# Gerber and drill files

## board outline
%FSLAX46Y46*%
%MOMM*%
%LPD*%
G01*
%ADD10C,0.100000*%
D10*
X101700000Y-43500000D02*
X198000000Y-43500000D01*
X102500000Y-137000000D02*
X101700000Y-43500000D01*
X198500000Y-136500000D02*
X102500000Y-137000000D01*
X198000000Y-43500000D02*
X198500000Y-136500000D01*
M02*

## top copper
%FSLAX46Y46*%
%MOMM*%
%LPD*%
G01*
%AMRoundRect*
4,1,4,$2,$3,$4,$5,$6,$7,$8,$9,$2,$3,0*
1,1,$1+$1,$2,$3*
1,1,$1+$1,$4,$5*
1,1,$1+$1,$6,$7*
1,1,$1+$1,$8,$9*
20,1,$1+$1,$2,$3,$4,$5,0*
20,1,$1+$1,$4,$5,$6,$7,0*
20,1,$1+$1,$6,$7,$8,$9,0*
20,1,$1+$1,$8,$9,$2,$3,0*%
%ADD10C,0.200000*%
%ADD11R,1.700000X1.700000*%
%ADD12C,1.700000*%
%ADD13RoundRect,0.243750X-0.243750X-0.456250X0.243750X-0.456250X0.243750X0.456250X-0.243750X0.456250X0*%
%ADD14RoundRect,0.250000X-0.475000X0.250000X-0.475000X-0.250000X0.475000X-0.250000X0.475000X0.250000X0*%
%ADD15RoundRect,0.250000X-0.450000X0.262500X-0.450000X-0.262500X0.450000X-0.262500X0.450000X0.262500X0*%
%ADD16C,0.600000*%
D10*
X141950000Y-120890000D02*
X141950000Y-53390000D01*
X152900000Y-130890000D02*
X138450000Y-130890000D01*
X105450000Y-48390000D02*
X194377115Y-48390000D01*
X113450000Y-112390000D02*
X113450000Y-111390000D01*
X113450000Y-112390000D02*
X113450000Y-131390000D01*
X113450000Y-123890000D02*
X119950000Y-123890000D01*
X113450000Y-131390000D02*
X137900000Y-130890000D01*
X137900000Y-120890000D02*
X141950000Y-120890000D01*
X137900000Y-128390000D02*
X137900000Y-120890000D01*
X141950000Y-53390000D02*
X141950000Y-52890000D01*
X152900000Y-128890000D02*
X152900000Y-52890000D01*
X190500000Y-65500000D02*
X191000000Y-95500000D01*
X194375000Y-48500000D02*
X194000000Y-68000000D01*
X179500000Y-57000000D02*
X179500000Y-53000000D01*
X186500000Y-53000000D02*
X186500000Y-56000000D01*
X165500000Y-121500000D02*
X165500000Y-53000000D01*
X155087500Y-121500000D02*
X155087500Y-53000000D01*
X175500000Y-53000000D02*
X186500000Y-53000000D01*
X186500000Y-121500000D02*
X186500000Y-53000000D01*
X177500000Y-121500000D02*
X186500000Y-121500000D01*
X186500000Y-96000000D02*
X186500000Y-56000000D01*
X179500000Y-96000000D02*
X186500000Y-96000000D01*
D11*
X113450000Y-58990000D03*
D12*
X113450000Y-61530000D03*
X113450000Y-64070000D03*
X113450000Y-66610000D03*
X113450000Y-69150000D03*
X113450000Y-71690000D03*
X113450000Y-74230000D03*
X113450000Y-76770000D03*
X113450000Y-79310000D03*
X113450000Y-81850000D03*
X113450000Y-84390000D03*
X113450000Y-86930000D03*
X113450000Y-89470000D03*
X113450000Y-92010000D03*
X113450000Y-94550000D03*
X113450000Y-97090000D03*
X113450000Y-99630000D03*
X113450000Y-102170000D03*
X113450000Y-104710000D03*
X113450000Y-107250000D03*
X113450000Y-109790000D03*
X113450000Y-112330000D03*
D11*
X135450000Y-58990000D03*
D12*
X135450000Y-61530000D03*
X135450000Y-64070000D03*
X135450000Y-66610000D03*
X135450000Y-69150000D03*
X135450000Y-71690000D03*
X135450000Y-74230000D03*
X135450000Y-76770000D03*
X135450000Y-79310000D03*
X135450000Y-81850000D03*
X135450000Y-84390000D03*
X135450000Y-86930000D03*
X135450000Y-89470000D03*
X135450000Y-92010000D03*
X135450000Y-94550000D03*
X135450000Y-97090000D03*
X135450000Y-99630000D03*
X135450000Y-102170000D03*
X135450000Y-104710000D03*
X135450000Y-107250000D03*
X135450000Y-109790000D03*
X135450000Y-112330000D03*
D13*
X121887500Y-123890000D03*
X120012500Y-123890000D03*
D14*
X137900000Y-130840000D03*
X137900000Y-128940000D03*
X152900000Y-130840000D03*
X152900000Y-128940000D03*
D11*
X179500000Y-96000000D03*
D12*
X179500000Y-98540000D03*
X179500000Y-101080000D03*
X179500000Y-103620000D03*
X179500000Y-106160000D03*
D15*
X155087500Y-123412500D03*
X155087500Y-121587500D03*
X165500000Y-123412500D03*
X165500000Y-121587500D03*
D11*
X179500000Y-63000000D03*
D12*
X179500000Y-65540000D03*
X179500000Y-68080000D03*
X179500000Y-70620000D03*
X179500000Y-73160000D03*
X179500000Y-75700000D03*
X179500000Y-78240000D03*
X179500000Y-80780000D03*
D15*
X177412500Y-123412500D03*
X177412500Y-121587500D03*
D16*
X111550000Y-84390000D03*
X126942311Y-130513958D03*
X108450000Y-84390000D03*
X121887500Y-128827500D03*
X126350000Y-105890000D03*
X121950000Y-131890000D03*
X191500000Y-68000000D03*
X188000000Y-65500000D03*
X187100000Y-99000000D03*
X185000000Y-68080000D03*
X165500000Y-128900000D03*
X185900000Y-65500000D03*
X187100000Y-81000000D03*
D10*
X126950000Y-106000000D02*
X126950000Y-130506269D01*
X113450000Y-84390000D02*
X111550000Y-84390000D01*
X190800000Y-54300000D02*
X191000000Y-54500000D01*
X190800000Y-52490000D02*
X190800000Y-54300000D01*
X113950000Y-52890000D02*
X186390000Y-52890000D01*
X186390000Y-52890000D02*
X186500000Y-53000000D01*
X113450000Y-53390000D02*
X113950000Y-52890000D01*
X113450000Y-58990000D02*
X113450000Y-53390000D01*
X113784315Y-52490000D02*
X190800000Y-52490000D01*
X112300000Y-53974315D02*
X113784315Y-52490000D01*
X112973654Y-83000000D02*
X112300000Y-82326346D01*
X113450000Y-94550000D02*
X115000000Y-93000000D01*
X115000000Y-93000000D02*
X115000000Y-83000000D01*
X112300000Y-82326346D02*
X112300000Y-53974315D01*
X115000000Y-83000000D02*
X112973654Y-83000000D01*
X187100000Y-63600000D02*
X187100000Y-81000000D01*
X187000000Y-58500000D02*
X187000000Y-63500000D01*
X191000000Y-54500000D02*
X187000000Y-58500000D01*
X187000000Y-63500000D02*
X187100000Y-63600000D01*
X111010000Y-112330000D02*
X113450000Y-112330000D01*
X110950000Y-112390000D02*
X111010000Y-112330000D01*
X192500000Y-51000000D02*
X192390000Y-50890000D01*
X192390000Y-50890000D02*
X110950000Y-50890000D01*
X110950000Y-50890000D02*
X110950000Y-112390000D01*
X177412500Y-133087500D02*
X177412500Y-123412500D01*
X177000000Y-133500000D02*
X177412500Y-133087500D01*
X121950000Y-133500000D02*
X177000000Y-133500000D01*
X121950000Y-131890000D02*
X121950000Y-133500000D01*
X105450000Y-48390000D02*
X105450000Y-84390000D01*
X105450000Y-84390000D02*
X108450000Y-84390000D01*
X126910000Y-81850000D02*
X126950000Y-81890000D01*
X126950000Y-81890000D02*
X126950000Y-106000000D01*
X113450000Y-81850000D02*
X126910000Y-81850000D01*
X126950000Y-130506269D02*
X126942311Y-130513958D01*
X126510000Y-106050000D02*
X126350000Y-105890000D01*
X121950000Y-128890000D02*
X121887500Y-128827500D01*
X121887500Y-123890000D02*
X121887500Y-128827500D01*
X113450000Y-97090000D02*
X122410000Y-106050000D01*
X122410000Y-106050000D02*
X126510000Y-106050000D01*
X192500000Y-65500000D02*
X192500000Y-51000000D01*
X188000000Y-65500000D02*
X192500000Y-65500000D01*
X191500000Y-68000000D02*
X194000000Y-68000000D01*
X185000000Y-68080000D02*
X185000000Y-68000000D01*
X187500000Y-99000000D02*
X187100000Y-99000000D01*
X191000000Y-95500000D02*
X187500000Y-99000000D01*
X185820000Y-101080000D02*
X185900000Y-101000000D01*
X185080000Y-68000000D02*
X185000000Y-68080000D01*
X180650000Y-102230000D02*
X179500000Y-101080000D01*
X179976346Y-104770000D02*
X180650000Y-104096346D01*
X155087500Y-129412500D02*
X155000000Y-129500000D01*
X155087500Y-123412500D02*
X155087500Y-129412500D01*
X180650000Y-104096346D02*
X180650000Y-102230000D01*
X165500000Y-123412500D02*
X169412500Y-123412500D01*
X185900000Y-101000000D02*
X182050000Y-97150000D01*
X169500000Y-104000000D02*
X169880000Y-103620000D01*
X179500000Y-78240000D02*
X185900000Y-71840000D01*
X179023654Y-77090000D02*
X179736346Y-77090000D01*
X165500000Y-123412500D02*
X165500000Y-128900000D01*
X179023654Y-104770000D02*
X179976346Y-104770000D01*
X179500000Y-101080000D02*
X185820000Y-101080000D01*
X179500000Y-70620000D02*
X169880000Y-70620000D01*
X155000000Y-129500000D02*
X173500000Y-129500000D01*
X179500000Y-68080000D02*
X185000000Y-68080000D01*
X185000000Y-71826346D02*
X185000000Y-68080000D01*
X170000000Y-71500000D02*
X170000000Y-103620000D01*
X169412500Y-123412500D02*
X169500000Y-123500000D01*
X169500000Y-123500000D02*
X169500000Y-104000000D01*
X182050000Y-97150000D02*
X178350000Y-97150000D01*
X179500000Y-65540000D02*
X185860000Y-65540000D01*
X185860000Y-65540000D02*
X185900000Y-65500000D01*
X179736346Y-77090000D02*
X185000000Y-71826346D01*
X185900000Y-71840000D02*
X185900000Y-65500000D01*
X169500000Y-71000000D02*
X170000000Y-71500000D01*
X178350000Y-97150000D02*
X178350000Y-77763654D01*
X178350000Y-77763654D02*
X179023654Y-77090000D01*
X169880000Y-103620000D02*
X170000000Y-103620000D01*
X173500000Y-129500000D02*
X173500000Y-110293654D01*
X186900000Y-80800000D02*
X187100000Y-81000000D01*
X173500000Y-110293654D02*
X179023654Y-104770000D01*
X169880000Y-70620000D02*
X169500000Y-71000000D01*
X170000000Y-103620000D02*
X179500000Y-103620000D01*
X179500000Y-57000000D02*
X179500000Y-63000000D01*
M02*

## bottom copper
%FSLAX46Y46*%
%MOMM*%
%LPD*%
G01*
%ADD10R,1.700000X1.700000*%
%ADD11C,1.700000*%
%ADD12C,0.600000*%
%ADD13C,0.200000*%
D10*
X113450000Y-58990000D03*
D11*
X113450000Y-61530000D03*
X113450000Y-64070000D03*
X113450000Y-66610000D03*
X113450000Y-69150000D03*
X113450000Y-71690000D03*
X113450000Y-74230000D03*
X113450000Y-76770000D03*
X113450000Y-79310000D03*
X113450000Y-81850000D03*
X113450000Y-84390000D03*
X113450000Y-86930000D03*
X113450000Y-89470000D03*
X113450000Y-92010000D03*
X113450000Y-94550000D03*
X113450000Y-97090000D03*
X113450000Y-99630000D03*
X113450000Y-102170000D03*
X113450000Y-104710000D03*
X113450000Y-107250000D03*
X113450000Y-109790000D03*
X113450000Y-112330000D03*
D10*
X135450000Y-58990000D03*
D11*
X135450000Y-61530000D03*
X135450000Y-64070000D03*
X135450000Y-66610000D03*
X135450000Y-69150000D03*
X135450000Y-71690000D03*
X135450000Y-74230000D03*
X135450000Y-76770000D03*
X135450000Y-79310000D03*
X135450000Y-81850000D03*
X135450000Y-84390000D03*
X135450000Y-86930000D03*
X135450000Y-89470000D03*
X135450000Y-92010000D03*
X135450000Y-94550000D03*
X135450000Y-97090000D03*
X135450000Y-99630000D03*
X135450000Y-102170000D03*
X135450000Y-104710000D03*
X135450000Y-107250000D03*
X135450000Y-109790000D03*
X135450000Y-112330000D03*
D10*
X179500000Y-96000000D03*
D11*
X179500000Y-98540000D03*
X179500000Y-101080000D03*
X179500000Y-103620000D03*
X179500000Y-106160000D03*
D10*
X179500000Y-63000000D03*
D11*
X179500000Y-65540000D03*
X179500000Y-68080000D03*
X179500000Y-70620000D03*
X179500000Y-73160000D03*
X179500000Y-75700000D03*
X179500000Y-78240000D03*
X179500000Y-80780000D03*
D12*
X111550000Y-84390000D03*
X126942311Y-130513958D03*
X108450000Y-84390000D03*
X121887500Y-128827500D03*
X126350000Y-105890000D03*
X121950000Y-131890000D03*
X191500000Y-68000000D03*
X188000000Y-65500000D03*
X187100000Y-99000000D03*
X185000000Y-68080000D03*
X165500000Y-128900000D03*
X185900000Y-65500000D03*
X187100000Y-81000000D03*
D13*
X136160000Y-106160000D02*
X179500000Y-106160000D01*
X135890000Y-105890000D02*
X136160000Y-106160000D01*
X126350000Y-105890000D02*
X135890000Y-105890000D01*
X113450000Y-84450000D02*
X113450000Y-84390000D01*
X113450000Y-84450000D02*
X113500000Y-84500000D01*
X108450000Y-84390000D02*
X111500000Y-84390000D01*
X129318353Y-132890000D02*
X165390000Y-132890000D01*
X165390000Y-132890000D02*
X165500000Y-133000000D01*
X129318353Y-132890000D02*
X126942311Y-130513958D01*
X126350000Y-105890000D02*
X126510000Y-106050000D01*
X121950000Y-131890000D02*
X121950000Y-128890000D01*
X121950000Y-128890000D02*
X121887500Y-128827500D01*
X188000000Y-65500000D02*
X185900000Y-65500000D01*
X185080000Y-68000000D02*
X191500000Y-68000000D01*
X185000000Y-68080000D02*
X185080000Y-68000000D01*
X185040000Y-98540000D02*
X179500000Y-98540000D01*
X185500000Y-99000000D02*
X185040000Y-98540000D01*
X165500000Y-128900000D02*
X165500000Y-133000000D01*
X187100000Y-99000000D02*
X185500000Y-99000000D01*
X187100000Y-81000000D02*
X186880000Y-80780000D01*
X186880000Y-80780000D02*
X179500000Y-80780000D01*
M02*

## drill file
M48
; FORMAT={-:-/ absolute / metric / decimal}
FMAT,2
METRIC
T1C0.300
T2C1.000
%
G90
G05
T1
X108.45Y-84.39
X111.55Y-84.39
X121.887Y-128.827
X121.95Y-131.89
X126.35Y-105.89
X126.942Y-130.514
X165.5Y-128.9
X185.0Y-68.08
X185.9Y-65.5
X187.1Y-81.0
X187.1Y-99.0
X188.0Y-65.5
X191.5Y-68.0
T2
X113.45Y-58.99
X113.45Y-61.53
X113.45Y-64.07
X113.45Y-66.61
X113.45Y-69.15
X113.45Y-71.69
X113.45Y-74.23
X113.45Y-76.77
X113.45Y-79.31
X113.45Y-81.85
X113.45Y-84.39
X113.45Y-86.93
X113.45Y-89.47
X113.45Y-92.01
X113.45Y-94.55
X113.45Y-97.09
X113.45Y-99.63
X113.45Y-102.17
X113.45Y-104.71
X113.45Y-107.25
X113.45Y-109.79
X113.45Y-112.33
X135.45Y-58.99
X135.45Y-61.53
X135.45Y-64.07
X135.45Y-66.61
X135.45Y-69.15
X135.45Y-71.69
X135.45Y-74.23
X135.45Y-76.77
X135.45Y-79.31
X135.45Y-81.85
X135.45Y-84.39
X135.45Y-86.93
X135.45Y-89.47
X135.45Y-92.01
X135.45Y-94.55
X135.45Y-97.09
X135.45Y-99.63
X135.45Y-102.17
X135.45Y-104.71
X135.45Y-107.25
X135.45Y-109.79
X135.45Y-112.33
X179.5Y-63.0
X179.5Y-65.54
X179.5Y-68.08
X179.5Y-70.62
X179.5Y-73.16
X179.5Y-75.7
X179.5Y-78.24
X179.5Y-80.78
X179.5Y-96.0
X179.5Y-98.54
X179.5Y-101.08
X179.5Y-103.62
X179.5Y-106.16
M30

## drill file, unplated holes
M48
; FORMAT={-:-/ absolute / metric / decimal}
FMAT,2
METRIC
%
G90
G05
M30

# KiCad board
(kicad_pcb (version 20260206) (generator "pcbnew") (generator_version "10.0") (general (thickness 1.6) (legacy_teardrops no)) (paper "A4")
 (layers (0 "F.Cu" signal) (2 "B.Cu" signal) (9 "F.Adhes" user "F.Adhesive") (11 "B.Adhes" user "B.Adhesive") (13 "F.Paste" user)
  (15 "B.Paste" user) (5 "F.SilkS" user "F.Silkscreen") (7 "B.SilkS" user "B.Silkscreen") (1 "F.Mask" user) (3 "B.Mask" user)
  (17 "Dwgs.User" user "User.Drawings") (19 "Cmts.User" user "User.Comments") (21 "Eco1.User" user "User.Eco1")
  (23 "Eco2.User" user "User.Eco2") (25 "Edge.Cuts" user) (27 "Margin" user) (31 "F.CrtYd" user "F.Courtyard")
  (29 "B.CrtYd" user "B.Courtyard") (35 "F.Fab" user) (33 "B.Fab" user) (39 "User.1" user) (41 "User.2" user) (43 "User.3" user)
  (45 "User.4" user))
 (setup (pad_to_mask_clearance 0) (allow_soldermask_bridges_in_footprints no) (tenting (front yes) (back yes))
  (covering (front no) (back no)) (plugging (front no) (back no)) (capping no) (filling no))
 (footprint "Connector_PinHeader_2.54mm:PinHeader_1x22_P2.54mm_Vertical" (layer "F.Cu") (at 135.45 58.99)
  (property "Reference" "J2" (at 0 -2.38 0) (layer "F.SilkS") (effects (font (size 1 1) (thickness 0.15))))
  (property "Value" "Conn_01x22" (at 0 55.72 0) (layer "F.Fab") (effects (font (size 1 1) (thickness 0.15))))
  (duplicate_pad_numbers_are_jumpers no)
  (pad "1" thru_hole rect (at 0 0) (size 1.7 1.7) (drill 1) (layers "*.Cu" "*.Mask") (remove_unused_layers no)
   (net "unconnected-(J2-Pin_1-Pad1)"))
  (pad "2" thru_hole circle (at 0 2.54) (size 1.7 1.7) (drill 1) (layers "*.Cu" "*.Mask") (remove_unused_layers no)
   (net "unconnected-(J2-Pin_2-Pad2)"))
  (pad "3" thru_hole circle (at 0 5.08) (size 1.7 1.7) (drill 1) (layers "*.Cu" "*.Mask") (remove_unused_layers no)
   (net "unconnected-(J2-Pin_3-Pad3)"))
  (pad "4" thru_hole circle (at 0 7.62) (size 1.7 1.7) (drill 1) (layers "*.Cu" "*.Mask") (remove_unused_layers no)
   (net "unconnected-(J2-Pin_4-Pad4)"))
  (pad "5" thru_hole circle (at 0 10.16) (size 1.7 1.7) (drill 1) (layers "*.Cu" "*.Mask") (remove_unused_layers no)
   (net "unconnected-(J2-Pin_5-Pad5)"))
  (pad "6" thru_hole circle (at 0 12.7) (size 1.7 1.7) (drill 1) (layers "*.Cu" "*.Mask") (remove_unused_layers no)
   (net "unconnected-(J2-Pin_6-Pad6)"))
  (pad "7" thru_hole circle (at 0 15.24) (size 1.7 1.7) (drill 1) (layers "*.Cu" "*.Mask") (remove_unused_layers no)
   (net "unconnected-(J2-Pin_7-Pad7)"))
  (pad "8" thru_hole circle (at 0 17.78) (size 1.7 1.7) (drill 1) (layers "*.Cu" "*.Mask") (remove_unused_layers no)
   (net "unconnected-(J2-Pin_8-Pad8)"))
  (pad "9" thru_hole circle (at 0 20.32) (size 1.7 1.7) (drill 1) (layers "*.Cu" "*.Mask") (remove_unused_layers no)
   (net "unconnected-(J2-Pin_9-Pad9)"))
  (pad "10" thru_hole circle (at 0 22.86) (size 1.7 1.7) (drill 1) (layers "*.Cu" "*.Mask") (remove_unused_layers no)
   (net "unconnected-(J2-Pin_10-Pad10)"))
  (pad "11" thru_hole circle (at 0 25.4) (size 1.7 1.7) (drill 1) (layers "*.Cu" "*.Mask") (remove_unused_layers no)
   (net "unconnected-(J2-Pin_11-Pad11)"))
  (pad "12" thru_hole circle (at 0 27.94) (size 1.7 1.7) (drill 1) (layers "*.Cu" "*.Mask") (remove_unused_layers no)
   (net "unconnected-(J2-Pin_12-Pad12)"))
  (pad "13" thru_hole circle (at 0 30.48) (size 1.7 1.7) (drill 1) (layers "*.Cu" "*.Mask") (remove_unused_layers no)
   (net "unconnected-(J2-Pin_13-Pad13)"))
  (pad "14" thru_hole circle (at 0 33.02) (size 1.7 1.7) (drill 1) (layers "*.Cu" "*.Mask") (remove_unused_layers no)
   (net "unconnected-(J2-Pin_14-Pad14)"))
  (pad "15" thru_hole circle (at 0 35.56) (size 1.7 1.7) (drill 1) (layers "*.Cu" "*.Mask") (remove_unused_layers no)
   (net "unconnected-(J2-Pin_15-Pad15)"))
  (pad "16" thru_hole circle (at 0 38.1) (size 1.7 1.7) (drill 1) (layers "*.Cu" "*.Mask") (remove_unused_layers no)
   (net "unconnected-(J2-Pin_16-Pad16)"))
  (pad "17" thru_hole circle (at 0 40.64) (size 1.7 1.7) (drill 1) (layers "*.Cu" "*.Mask") (remove_unused_layers no)
   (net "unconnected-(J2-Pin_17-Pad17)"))
  (pad "18" thru_hole circle (at 0 43.18) (size 1.7 1.7) (drill 1) (layers "*.Cu" "*.Mask") (remove_unused_layers no)
   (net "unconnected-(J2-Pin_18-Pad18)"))
  (pad "19" thru_hole circle (at 0 45.72) (size 1.7 1.7) (drill 1) (layers "*.Cu" "*.Mask") (remove_unused_layers no)
   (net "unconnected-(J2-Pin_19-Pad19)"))
  (pad "20" thru_hole circle (at 0 48.26) (size 1.7 1.7) (drill 1) (layers "*.Cu" "*.Mask") (remove_unused_layers no)
   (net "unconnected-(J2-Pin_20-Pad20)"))
  (pad "21" thru_hole circle (at 0 50.8) (size 1.7 1.7) (drill 1) (layers "*.Cu" "*.Mask") (remove_unused_layers no)
   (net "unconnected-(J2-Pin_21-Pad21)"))
  (pad "22" thru_hole circle (at 0 53.34) (size 1.7 1.7) (drill 1) (layers "*.Cu" "*.Mask") (remove_unused_layers no)
   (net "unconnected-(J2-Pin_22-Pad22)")))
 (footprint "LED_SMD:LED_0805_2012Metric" (layer "F.Cu") (at 120.95 123.89)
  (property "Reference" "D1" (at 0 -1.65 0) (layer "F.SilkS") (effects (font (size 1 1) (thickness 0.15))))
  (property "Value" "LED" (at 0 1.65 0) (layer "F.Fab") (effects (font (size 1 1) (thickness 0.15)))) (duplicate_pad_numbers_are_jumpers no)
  (pad "1" smd roundrect (at -0.9375 0) (size 0.975 1.4) (layers "F.Cu" "F.Mask" "F.Paste") (roundrect_rratio 0.25) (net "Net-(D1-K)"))
  (pad "2" smd roundrect (at 0.9375 0) (size 0.975 1.4) (layers "F.Cu" "F.Mask" "F.Paste") (roundrect_rratio 0.25) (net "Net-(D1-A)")))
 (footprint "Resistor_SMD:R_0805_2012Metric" (layer "F.Cu") (at 165.5 122.5 -90)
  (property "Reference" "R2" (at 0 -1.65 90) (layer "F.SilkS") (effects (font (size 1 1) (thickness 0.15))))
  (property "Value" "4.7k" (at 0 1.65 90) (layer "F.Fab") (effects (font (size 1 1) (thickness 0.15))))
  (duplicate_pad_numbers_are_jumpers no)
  (pad "1" smd roundrect (at -0.9125 0 270) (size 1.025 1.4) (layers "F.Cu" "F.Mask" "F.Paste") (roundrect_rratio 0.243902) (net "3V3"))
  (pad "2" smd roundrect (at 0.9125 0 270) (size 1.025 1.4) (layers "F.Cu" "F.Mask" "F.Paste") (roundrect_rratio 0.243902)
   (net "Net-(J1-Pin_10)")))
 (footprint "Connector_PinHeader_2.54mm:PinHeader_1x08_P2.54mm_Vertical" (layer "F.Cu") (at 179.5 63)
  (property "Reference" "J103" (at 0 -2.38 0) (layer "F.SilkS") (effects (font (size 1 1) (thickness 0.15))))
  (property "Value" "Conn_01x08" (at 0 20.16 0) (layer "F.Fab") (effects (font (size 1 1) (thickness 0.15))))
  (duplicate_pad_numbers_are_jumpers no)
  (pad "1" thru_hole rect (at 0 0) (size 1.7 1.7) (drill 1) (layers "*.Cu" "*.Mask") (remove_unused_layers no) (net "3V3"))
  (pad "2" thru_hole circle (at 0 2.54) (size 1.7 1.7) (drill 1) (layers "*.Cu" "*.Mask") (remove_unused_layers no) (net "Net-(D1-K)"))
  (pad "3" thru_hole circle (at 0 5.08) (size 1.7 1.7) (drill 1) (layers "*.Cu" "*.Mask") (remove_unused_layers no) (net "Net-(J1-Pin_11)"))
  (pad "4" thru_hole circle (at 0 7.62) (size 1.7 1.7) (drill 1) (layers "*.Cu" "*.Mask") (remove_unused_layers no) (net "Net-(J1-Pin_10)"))
  (pad "5" thru_hole circle (at 0 10.16) (size 1.7 1.7) (drill 1) (layers "*.Cu" "*.Mask") (remove_unused_layers no)
   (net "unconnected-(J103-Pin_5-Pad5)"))
  (pad "6" thru_hole circle (at 0 12.7) (size 1.7 1.7) (drill 1) (layers "*.Cu" "*.Mask") (remove_unused_layers no)
   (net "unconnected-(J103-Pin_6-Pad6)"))
  (pad "7" thru_hole circle (at 0 15.24) (size 1.7 1.7) (drill 1) (layers "*.Cu" "*.Mask") (remove_unused_layers no) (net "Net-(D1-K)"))
  (pad "8" thru_hole circle (at 0 17.78) (size 1.7 1.7) (drill 1) (layers "*.Cu" "*.Mask") (remove_unused_layers no) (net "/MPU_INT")))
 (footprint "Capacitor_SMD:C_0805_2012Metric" (layer "F.Cu") (at 137.9 129.89 -90)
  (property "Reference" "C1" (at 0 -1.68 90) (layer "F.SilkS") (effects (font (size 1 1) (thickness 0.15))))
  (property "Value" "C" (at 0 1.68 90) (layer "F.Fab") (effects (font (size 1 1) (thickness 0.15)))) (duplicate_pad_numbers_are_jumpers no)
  (pad "1" smd roundrect (at -0.95 0 270) (size 1 1.45) (layers "F.Cu" "F.Mask" "F.Paste") (roundrect_rratio 0.25) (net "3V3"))
  (pad "2" smd roundrect (at 0.95 0 270) (size 1 1.45) (layers "F.Cu" "F.Mask" "F.Paste") (roundrect_rratio 0.25) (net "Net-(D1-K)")))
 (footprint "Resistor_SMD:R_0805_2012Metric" (layer "F.Cu") (at 177.4125 122.5 -90)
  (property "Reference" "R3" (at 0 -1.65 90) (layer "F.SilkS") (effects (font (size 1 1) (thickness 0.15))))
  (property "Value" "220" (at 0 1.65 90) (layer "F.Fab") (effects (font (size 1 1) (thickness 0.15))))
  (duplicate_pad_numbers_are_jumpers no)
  (pad "1" smd roundrect (at -0.9125 0 270) (size 1.025 1.4) (layers "F.Cu" "F.Mask" "F.Paste") (roundrect_rratio 0.243902) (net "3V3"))
  (pad "2" smd roundrect (at 0.9125 0 270) (size 1.025 1.4) (layers "F.Cu" "F.Mask" "F.Paste") (roundrect_rratio 0.243902)
   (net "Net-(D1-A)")))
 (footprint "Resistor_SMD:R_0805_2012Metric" (layer "F.Cu") (at 155.0875 122.5 -90)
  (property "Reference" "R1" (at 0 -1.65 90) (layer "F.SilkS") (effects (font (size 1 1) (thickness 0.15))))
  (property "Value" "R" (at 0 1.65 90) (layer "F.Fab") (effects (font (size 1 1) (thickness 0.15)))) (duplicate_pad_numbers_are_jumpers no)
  (pad "1" smd roundrect (at -0.9125 0 270) (size 1.025 1.4) (layers "F.Cu" "F.Mask" "F.Paste") (roundrect_rratio 0.243902) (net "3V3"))
  (pad "2" smd roundrect (at 0.9125 0 270) (size 1.025 1.4) (layers "F.Cu" "F.Mask" "F.Paste") (roundrect_rratio 0.243902)
   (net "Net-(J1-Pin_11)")))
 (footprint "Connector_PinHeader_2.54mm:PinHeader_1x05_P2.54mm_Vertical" (layer "F.Cu") (at 179.5 96)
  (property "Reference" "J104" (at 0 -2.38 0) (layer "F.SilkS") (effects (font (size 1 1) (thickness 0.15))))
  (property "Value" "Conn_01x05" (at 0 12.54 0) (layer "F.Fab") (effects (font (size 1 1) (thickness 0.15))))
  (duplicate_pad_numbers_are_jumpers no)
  (pad "1" thru_hole rect (at 0 0) (size 1.7 1.7) (drill 1) (layers "*.Cu" "*.Mask") (remove_unused_layers no) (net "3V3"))
  (pad "2" thru_hole circle (at 0 2.54) (size 1.7 1.7) (drill 1) (layers "*.Cu" "*.Mask") (remove_unused_layers no) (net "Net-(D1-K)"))
  (pad "3" thru_hole circle (at 0 5.08) (size 1.7 1.7) (drill 1) (layers "*.Cu" "*.Mask") (remove_unused_layers no) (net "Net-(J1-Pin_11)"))
  (pad "4" thru_hole circle (at 0 7.62) (size 1.7 1.7) (drill 1) (layers "*.Cu" "*.Mask") (remove_unused_layers no) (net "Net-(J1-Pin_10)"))
  (pad "5" thru_hole circle (at 0 10.16) (size 1.7 1.7) (drill 1) (layers "*.Cu" "*.Mask") (remove_unused_layers no) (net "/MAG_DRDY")))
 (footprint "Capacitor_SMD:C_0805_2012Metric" (layer "F.Cu") (at 152.9 129.89 -90)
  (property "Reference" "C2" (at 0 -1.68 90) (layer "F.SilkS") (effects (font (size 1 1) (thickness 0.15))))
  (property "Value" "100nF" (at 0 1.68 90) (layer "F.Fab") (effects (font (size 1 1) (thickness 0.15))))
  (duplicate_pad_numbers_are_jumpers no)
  (pad "1" smd roundrect (at -0.95 0 270) (size 1 1.45) (layers "F.Cu" "F.Mask" "F.Paste") (roundrect_rratio 0.25) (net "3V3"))
  (pad "2" smd roundrect (at 0.95 0 270) (size 1 1.45) (layers "F.Cu" "F.Mask" "F.Paste") (roundrect_rratio 0.25) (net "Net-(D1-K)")))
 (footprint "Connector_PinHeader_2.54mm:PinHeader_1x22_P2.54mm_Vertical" (layer "F.Cu") (at 113.45 58.99)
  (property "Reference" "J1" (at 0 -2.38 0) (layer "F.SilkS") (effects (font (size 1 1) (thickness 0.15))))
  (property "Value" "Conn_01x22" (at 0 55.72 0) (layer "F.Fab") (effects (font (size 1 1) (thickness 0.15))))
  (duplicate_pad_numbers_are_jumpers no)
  (pad "1" thru_hole rect (at 0 0) (size 1.7 1.7) (drill 1) (layers "*.Cu" "*.Mask") (remove_unused_layers no) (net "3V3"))
  (pad "2" thru_hole circle (at 0 2.54) (size 1.7 1.7) (drill 1) (layers "*.Cu" "*.Mask") (remove_unused_layers no)
   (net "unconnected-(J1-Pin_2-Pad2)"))
  (pad "3" thru_hole circle (at 0 5.08) (size 1.7 1.7) (drill 1) (layers "*.Cu" "*.Mask") (remove_unused_layers no)
   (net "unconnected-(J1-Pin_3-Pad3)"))
  (pad "4" thru_hole circle (at 0 7.62) (size 1.7 1.7) (drill 1) (layers "*.Cu" "*.Mask") (remove_unused_layers no)
   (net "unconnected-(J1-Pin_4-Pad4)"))
  (pad "5" thru_hole circle (at 0 10.16) (size 1.7 1.7) (drill 1) (layers "*.Cu" "*.Mask") (remove_unused_layers no)
   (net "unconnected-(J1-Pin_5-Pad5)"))
  (pad "6" thru_hole circle (at 0 12.7) (size 1.7 1.7) (drill 1) (layers "*.Cu" "*.Mask") (remove_unused_layers no)
   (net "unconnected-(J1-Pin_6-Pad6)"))
  (pad "7" thru_hole circle (at 0 15.24) (size 1.7 1.7) (drill 1) (layers "*.Cu" "*.Mask") (remove_unused_layers no)
   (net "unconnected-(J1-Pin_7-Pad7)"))
  (pad "8" thru_hole circle (at 0 17.78) (size 1.7 1.7) (drill 1) (layers "*.Cu" "*.Mask") (remove_unused_layers no)
   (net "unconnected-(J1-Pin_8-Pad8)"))
  (pad "9" thru_hole circle (at 0 20.32) (size 1.7 1.7) (drill 1) (layers "*.Cu" "*.Mask") (remove_unused_layers no)
   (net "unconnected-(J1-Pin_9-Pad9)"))
  (pad "10" thru_hole circle (at 0 22.86) (size 1.7 1.7) (drill 1) (layers "*.Cu" "*.Mask") (remove_unused_layers no)
   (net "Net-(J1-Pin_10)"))
  (pad "11" thru_hole circle (at 0 25.4) (size 1.7 1.7) (drill 1) (layers "*.Cu" "*.Mask") (remove_unused_layers no) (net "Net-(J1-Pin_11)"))
  (pad "12" thru_hole circle (at 0 27.94) (size 1.7 1.7) (drill 1) (layers "*.Cu" "*.Mask") (remove_unused_layers no)
   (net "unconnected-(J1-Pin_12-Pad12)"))
  (pad "13" thru_hole circle (at 0 30.48) (size 1.7 1.7) (drill 1) (layers "*.Cu" "*.Mask") (remove_unused_layers no)
   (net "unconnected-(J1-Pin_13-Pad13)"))
  (pad "14" thru_hole circle (at 0 33.02) (size 1.7 1.7) (drill 1) (layers "*.Cu" "*.Mask") (remove_unused_layers no)
   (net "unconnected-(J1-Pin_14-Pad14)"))
  (pad "15" thru_hole circle (at 0 35.56) (size 1.7 1.7) (drill 1) (layers "*.Cu" "*.Mask") (remove_unused_layers no) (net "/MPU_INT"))
  (pad "16" thru_hole circle (at 0 38.1) (size 1.7 1.7) (drill 1) (layers "*.Cu" "*.Mask") (remove_unused_layers no) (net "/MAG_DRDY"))
  (pad "17" thru_hole circle (at 0 40.64) (size 1.7 1.7) (drill 1) (layers "*.Cu" "*.Mask") (remove_unused_layers no)
   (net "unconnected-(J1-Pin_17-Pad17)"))
  (pad "18" thru_hole circle (at 0 43.18) (size 1.7 1.7) (drill 1) (layers "*.Cu" "*.Mask") (remove_unused_layers no)
   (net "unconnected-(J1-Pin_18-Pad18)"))
  (pad "19" thru_hole circle (at 0 45.72) (size 1.7 1.7) (drill 1) (layers "*.Cu" "*.Mask") (remove_unused_layers no)
   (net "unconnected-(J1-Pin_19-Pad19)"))
  (pad "20" thru_hole circle (at 0 48.26) (size 1.7 1.7) (drill 1) (layers "*.Cu" "*.Mask") (remove_unused_layers no)
   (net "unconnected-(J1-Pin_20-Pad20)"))
  (pad "21" thru_hole circle (at 0 50.8) (size 1.7 1.7) (drill 1) (layers "*.Cu" "*.Mask") (remove_unused_layers no)
   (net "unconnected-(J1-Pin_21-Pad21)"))
  (pad "22" thru_hole circle (at 0 53.34) (size 1.7 1.7) (drill 1) (layers "*.Cu" "*.Mask") (remove_unused_layers no) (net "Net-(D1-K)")))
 (gr_line (start 105.45 48.39) (end 194.377115 48.39) (stroke (width 0.2) (type default)) (layer "F.Cu") (net "Net-(J1-Pin_11)"))
 (gr_line (start 113.45 112.39) (end 113.45 111.39) (stroke (width 0.2) (type default)) (layer "F.Cu") (net "Net-(D1-K)"))
 (gr_line (start 113.45 112.39) (end 113.45 131.39) (stroke (width 0.2) (type default)) (layer "F.Cu") (net "Net-(D1-K)"))
 (gr_line (start 113.45 123.89) (end 119.95 123.89) (stroke (width 0.2) (type default)) (layer "F.Cu") (net "Net-(D1-K)"))
 (gr_line (start 113.45 131.39) (end 137.9 130.89) (stroke (width 0.2) (type default)) (layer "F.Cu") (net "Net-(D1-K)"))
 (gr_line (start 137.9 120.89) (end 141.95 120.89) (stroke (width 0.2) (type default)) (layer "F.Cu") (net "3V3"))
 (gr_line (start 137.9 128.39) (end 137.9 120.89) (stroke (width 0.2) (type default)) (layer "F.Cu") (net "3V3"))
 (gr_line (start 141.95 53.39) (end 141.95 52.89) (stroke (width 0.2) (type default)) (layer "F.Cu") (net "3V3"))
 (gr_line (start 141.95 120.89) (end 141.95 53.39) (stroke (width 0.2) (type default)) (layer "F.Cu") (net "3V3"))
 (gr_line (start 152.9 128.89) (end 152.9 52.89) (stroke (width 0.2) (type default)) (layer "F.Cu") (net "3V3"))
 (gr_line (start 152.9 130.89) (end 138.45 130.89) (stroke (width 0.2) (type default)) (layer "F.Cu") (net "Net-(D1-K)"))
 (gr_line (start 155.0875 121.5) (end 155.0875 53) (stroke (width 0.2) (type default)) (layer "F.Cu") (net "3V3"))
 (gr_line (start 165.5 121.5) (end 165.5 53) (stroke (width 0.2) (type default)) (layer "F.Cu") (net "3V3"))
 (gr_line (start 177.5 121.5) (end 186.5 121.5) (stroke (width 0.2) (type default)) (layer "F.Cu") (net "3V3"))
 (gr_line (start 179.5 57) (end 179.5 53) (stroke (width 0.2) (type default)) (layer "F.Cu") (net "3V3"))
 (gr_line (start 179.5 96) (end 186.5 96) (stroke (width 0.2) (type default)) (layer "F.Cu") (net "3V3"))
 (gr_line (start 186.5 53) (end 186.5 56) (stroke (width 0.2) (type default)) (layer "F.Cu") (net "3V3"))
 (gr_line (start 186.5 96) (end 186.5 56) (stroke (width 0.2) (type default)) (layer "F.Cu") (net "3V3"))
 (gr_line (start 186.5 121.5) (end 186.5 53) (stroke (width 0.2) (type default)) (layer "F.Cu") (net "3V3"))
 (gr_line (start 190.5 65.5) (end 191 95.5) (stroke (width 0.2) (type default)) (layer "F.Cu") (net "Net-(D1-K)"))
 (gr_line (start 194.375 48.5) (end 194 68) (stroke (width 0.2) (type default)) (layer "F.Cu") (net "Net-(J1-Pin_11)"))
 (gr_line (start 101.7 43.5) (end 198 43.5) (stroke (width 0.1) (type default)) (layer "Edge.Cuts"))
 (gr_line (start 102.5 137) (end 101.7 43.5) (stroke (width 0.1) (type default)) (layer "Edge.Cuts"))
 (gr_line (start 198 43.5) (end 198.5 136.5) (stroke (width 0.1) (type default)) (layer "Edge.Cuts"))
 (gr_line (start 198.5 136.5) (end 102.5 137) (stroke (width 0.1) (type default)) (layer "Edge.Cuts"))
 (segment (start 110.95 112.39) (end 111.01 112.33) (width 0.2) (layer "F.Cu") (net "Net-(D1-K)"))
 (segment (start 192.5 51) (end 192.39 50.89) (width 0.2) (layer "F.Cu") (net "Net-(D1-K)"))
 (segment (start 192.5 65.5) (end 192.5 51) (width 0.2) (layer "F.Cu") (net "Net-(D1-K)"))
 (segment (start 191 95.5) (end 187.5 99) (width 0.2) (layer "F.Cu") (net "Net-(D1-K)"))
 (segment (start 188 65.5) (end 192.5 65.5) (width 0.2) (layer "F.Cu") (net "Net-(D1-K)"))
 (segment (start 192.39 50.89) (end 110.95 50.89) (width 0.2) (layer "F.Cu") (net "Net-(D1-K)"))
 (segment (start 179.5 65.54) (end 185.86 65.54) (width 0.2) (layer "F.Cu") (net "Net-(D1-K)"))
 (segment (start 179.5 78.24) (end 185.9 71.84) (width 0.2) (layer "F.Cu") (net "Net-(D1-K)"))
 (segment (start 187.5 99) (end 187.1 99) (width 0.2) (layer "F.Cu") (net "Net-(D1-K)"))
 (segment (start 111.01 112.33) (end 113.45 112.33) (width 0.2) (layer "F.Cu") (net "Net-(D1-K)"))
 (segment (start 110.95 50.89) (end 110.95 112.39) (width 0.2) (layer "F.Cu") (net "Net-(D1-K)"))
 (segment (start 185.86 65.54) (end 185.9 65.5) (width 0.2) (layer "F.Cu") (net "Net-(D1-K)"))
 (segment (start 185.9 71.84) (end 185.9 65.5) (width 0.2) (layer "F.Cu") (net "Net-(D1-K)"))
 (via (at 188 65.5) (size 0.6) (drill 0.3) (layers "F.Cu" "B.Cu") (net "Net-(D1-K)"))
 (via (at 185.9 65.5) (size 0.6) (drill 0.3) (layers "F.Cu" "B.Cu") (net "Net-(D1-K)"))
 (via (at 187.1 99) (size 0.6) (drill 0.3) (layers "F.Cu" "B.Cu") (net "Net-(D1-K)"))
 (segment (start 188 65.5) (end 185.9 65.5) (width 0.2) (layer "B.Cu") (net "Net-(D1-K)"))
 (segment (start 185.04 98.54) (end 179.5 98.54) (width 0.2) (layer "B.Cu") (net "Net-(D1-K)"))
 (segment (start 185.5 99) (end 185.04 98.54) (width 0.2) (layer "B.Cu") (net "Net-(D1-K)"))
 (segment (start 187.1 99) (end 185.5 99) (width 0.2) (layer "B.Cu") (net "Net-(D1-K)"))
 (segment (start 121.8875 123.89) (end 121.8875 128.8275) (width 0.2) (layer "F.Cu") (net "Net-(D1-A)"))
 (segment (start 121.95 133.5) (end 177 133.5) (width 0.2) (layer "F.Cu") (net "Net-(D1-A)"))
 (segment (start 121.95 128.89) (end 121.8875 128.8275) (width 0.2) (layer "F.Cu") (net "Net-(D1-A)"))
 (segment (start 177.4125 133.0875) (end 177.4125 123.4125) (width 0.2) (layer "F.Cu") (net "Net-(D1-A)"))
 (segment (start 177 133.5) (end 177.4125 133.0875) (width 0.2) (layer "F.Cu") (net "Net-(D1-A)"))
 (segment (start 121.95 131.89) (end 121.95 133.5) (width 0.2) (layer "F.Cu") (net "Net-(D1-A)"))
 (via (at 121.8875 128.8275) (size 0.6) (drill 0.3) (layers "F.Cu" "B.Cu") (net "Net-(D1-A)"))
 (via (at 121.95 131.89) (size 0.6) (drill 0.3) (layers "F.Cu" "B.Cu") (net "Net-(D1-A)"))
 (segment (start 121.95 128.89) (end 121.8875 128.8275) (width 0.2) (layer "B.Cu") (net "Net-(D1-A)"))
 (segment (start 121.95 131.89) (end 121.95 128.89) (width 0.2) (layer "B.Cu") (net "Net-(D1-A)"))
 (segment (start 186.39 52.89) (end 186.5 53) (width 0.2) (layer "F.Cu") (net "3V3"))
 (segment (start 113.95 52.89) (end 186.39 52.89) (width 0.2) (layer "F.Cu") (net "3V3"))
 (segment (start 179.5 57) (end 179.5 63) (width 0.2) (layer "F.Cu") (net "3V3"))
 (segment (start 113.45 58.99) (end 113.45 53.39) (width 0.2) (layer "F.Cu") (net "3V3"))
 (segment (start 113.45 53.39) (end 113.95 52.89) (width 0.2) (layer "F.Cu") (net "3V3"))
 (segment (start 179.5 70.62) (end 169.88 70.62) (width 0.2) (layer "F.Cu") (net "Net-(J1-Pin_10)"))
 (segment (start 169.88 103.62) (end 170 103.62) (width 0.2) (layer "F.Cu") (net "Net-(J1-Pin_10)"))
 (segment (start 169.5 71) (end 170 71.5) (width 0.2) (layer "F.Cu") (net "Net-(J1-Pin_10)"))
 (segment (start 126.91 81.85) (end 126.95 81.89) (width 0.2) (layer "F.Cu") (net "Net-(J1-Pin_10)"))
 (segment (start 165.5 123.4125) (end 165.5 128.9) (width 0.2) (layer "F.Cu") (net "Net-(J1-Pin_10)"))
 (segment (start 169.5 123.5) (end 169.5 104) (width 0.2) (layer "F.Cu") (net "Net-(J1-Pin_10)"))
 (segment (start 165.5 123.4125) (end 169.4125 123.4125) (width 0.2) (layer "F.Cu") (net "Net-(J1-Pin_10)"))
 (segment (start 126.95 130.506269) (end 126.942311 130.513958) (width 0.2) (layer "F.Cu") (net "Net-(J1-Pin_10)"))
 (segment (start 169.5 104) (end 169.88 103.62) (width 0.2) (layer "F.Cu") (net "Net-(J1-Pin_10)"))
 (segment (start 113.45 81.85) (end 126.91 81.85) (width 0.2) (layer "F.Cu") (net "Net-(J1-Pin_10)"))
 (segment (start 169.4125 123.4125) (end 169.5 123.5) (width 0.2) (layer "F.Cu") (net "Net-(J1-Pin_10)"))
 (segment (start 169.88 70.62) (end 169.5 71) (width 0.2) (layer "F.Cu") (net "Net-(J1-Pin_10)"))
 (segment (start 126.95 106) (end 126.95 130.506269) (width 0.2) (layer "F.Cu") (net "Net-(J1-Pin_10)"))
 (segment (start 126.95 81.89) (end 126.95 106) (width 0.2) (layer "F.Cu") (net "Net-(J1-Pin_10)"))
 (segment (start 170 71.5) (end 170 103.62) (width 0.2) (layer "F.Cu") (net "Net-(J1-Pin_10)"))
 (segment (start 170 103.62) (end 179.5 103.62) (width 0.2) (layer "F.Cu") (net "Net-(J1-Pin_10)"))
 (via (at 165.5 128.9) (size 0.6) (drill 0.3) (layers "F.Cu" "B.Cu") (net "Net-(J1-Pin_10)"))
 (via (at 126.942311 130.513958) (size 0.6) (drill 0.3) (layers "F.Cu" "B.Cu") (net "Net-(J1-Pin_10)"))
 (segment (start 129.318353 132.89) (end 165.39 132.89) (width 0.2) (layer "B.Cu") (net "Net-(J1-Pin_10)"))
 (segment (start 129.318353 132.89) (end 126.942311 130.513958) (width 0.2) (layer "B.Cu") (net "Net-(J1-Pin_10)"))
 (segment (start 165.5 128.9) (end 165.5 133) (width 0.2) (layer "B.Cu") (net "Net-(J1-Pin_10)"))
 (segment (start 165.39 132.89) (end 165.5 133) (width 0.2) (layer "B.Cu") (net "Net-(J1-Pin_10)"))
 (segment (start 180.65 102.23) (end 179.5 101.08) (width 0.2) (layer "F.Cu") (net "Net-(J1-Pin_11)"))
 (segment (start 185 68.08) (end 185 68) (width 0.2) (layer "F.Cu") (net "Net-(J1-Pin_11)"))
 (segment (start 185.82 101.08) (end 185.9 101) (width 0.2) (layer "F.Cu") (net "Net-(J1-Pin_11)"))
 (segment (start 179.976346 104.77) (end 180.65 104.096346) (width 0.2) (layer "F.Cu") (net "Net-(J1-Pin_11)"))
 (segment (start 155.0875 129.4125) (end 155 129.5) (width 0.2) (layer "F.Cu") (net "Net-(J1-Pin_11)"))
 (segment (start 185.08 68) (end 185 68.08) (width 0.2) (layer "F.Cu") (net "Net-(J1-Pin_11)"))
 (segment (start 178.35 97.15) (end 178.35 77.763654) (width 0.2) (layer "F.Cu") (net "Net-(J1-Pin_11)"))
 (segment (start 185.9 101) (end 182.05 97.15) (width 0.2) (layer "F.Cu") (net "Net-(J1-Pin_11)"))
 (segment (start 155 129.5) (end 173.5 129.5) (width 0.2) (layer "F.Cu") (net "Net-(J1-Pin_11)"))
 (segment (start 105.45 48.39) (end 105.45 84.39) (width 0.2) (layer "F.Cu") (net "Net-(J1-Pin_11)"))
 (segment (start 179.023654 77.09) (end 179.736346 77.09) (width 0.2) (layer "F.Cu") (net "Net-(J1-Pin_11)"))
 (segment (start 105.45 84.39) (end 108.45 84.39) (width 0.2) (layer "F.Cu") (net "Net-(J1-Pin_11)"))
 (segment (start 179.023654 104.77) (end 179.976346 104.77) (width 0.2) (layer "F.Cu") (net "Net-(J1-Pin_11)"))
 (segment (start 178.35 77.763654) (end 179.023654 77.09) (width 0.2) (layer "F.Cu") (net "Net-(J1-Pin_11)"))
 (segment (start 173.5 110.293654) (end 179.023654 104.77) (width 0.2) (layer "F.Cu") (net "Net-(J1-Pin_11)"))
 (segment (start 113.45 84.39) (end 111.55 84.39) (width 0.2) (layer "F.Cu") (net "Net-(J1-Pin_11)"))
 (segment (start 191.5 68) (end 194 68) (width 0.2) (layer "F.Cu") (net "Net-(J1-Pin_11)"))
 (segment (start 179.736346 77.09) (end 185 71.826346) (width 0.2) (layer "F.Cu") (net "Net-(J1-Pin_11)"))
 (segment (start 173.5 129.5) (end 173.5 110.293654) (width 0.2) (layer "F.Cu") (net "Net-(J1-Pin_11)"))
 (segment (start 155.0875 123.4125) (end 155.0875 129.4125) (width 0.2) (layer "F.Cu") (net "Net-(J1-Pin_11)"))
 (segment (start 179.5 68.08) (end 185 68.08) (width 0.2) (layer "F.Cu") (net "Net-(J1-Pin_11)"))
 (segment (start 185 71.826346) (end 185 68.08) (width 0.2) (layer "F.Cu") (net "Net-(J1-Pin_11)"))
 (segment (start 180.65 104.096346) (end 180.65 102.23) (width 0.2) (layer "F.Cu") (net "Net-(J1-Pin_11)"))
 (segment (start 182.05 97.15) (end 178.35 97.15) (width 0.2) (layer "F.Cu") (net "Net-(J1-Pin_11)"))
 (segment (start 179.5 101.08) (end 185.82 101.08) (width 0.2) (layer "F.Cu") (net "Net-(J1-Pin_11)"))
 (via (at 111.55 84.39) (size 0.6) (drill 0.3) (layers "F.Cu" "B.Cu") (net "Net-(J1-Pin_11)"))
 (via (at 108.45 84.39) (size 0.6) (drill 0.3) (layers "F.Cu" "B.Cu") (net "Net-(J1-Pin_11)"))
 (via (at 185 68.08) (size 0.6) (drill 0.3) (layers "F.Cu" "B.Cu") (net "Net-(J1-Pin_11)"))
 (via (at 191.5 68) (size 0.6) (drill 0.3) (layers "F.Cu" "B.Cu") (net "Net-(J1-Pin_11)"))
 (segment (start 113.45 84.45) (end 113.5 84.5) (width 0.2) (layer "B.Cu") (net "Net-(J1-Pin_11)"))
 (segment (start 108.45 84.39) (end 111.5 84.39) (width 0.2) (layer "B.Cu") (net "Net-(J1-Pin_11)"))
 (segment (start 185.08 68) (end 191.5 68) (width 0.2) (layer "B.Cu") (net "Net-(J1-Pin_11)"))
 (segment (start 185 68.08) (end 185.08 68) (width 0.2) (layer "B.Cu") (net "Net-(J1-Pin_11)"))
 (segment (start 113.45 84.45) (end 113.45 84.39) (width 0.2) (layer "B.Cu") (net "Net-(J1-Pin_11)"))
 (segment (start 187.1 63.6) (end 187.1 81) (width 0.2) (layer "F.Cu") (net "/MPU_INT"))
 (segment (start 115 93) (end 115 83) (width 0.2) (layer "F.Cu") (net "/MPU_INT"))
 (segment (start 112.3 82.326346) (end 112.3 53.974315) (width 0.2) (layer "F.Cu") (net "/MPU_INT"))
 (segment (start 187 58.5) (end 187 63.5) (width 0.2) (layer "F.Cu") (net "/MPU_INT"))
 (segment (start 190.5 52.5) (end 190.5 55) (width 0.2) (layer "F.Cu") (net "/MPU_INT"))
 (segment (start 113.45 94.55) (end 115 93) (width 0.2) (layer "F.Cu") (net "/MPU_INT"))
 (segment (start 187 63.5) (end 187.1 63.6) (width 0.2) (layer "F.Cu") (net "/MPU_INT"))
 (segment (start 186.9 80.8) (end 187.1 81) (width 0.2) (layer "F.Cu") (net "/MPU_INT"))
 (segment (start 113.784315 52.49) (end 190.49 52.49) (width 0.2) (layer "F.Cu") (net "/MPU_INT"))
 (segment (start 190.49 52.49) (end 190.5 52.5) (width 0.2) (layer "F.Cu") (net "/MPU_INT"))
 (segment (start 115 83) (end 112.973654 83) (width 0.2) (layer "F.Cu") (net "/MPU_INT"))
 (segment (start 112.973654 83) (end 112.3 82.326346) (width 0.2) (layer "F.Cu") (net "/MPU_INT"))
 (segment (start 112.3 53.974315) (end 113.784315 52.49) (width 0.2) (layer "F.Cu") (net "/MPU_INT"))
 (segment (start 190.5 55) (end 187 58.5) (width 0.2) (layer "F.Cu") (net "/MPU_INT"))
 (via (at 187.1 81) (size 0.6) (drill 0.3) (layers "F.Cu" "B.Cu") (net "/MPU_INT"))
 (segment (start 187.1 81) (end 186.88 80.78) (width 0.2) (layer "B.Cu") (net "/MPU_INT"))
 (segment (start 186.88 80.78) (end 179.5 80.78) (width 0.2) (layer "B.Cu") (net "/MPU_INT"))
 (segment (start 126.51 106.05) (end 126.35 105.89) (width 0.2) (layer "F.Cu") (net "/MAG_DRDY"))
 (segment (start 113.45 97.09) (end 122.41 106.05) (width 0.2) (layer "F.Cu") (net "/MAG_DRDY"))
 (segment (start 122.41 106.05) (end 126.51 106.05) (width 0.2) (layer "F.Cu") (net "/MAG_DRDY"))
 (via (at 126.35 105.89) (size 0.6) (drill 0.3) (layers "F.Cu" "B.Cu") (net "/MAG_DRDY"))
 (segment (start 126.35 105.89) (end 135.89 105.89) (width 0.2) (layer "B.Cu") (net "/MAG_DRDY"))
 (segment (start 136.16 106.16) (end 179.5 106.16) (width 0.2) (layer "B.Cu") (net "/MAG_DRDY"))
 (segment (start 135.89 105.89) (end 136.16 106.16) (width 0.2) (layer "B.Cu") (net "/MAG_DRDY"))
 (segment (start 126.35 105.89) (end 126.51 106.05) (width 0.2) (layer "B.Cu") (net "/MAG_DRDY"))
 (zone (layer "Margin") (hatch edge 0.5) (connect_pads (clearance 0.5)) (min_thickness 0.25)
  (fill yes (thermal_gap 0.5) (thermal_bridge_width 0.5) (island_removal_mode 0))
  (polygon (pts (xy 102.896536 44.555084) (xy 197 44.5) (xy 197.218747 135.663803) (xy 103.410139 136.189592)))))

